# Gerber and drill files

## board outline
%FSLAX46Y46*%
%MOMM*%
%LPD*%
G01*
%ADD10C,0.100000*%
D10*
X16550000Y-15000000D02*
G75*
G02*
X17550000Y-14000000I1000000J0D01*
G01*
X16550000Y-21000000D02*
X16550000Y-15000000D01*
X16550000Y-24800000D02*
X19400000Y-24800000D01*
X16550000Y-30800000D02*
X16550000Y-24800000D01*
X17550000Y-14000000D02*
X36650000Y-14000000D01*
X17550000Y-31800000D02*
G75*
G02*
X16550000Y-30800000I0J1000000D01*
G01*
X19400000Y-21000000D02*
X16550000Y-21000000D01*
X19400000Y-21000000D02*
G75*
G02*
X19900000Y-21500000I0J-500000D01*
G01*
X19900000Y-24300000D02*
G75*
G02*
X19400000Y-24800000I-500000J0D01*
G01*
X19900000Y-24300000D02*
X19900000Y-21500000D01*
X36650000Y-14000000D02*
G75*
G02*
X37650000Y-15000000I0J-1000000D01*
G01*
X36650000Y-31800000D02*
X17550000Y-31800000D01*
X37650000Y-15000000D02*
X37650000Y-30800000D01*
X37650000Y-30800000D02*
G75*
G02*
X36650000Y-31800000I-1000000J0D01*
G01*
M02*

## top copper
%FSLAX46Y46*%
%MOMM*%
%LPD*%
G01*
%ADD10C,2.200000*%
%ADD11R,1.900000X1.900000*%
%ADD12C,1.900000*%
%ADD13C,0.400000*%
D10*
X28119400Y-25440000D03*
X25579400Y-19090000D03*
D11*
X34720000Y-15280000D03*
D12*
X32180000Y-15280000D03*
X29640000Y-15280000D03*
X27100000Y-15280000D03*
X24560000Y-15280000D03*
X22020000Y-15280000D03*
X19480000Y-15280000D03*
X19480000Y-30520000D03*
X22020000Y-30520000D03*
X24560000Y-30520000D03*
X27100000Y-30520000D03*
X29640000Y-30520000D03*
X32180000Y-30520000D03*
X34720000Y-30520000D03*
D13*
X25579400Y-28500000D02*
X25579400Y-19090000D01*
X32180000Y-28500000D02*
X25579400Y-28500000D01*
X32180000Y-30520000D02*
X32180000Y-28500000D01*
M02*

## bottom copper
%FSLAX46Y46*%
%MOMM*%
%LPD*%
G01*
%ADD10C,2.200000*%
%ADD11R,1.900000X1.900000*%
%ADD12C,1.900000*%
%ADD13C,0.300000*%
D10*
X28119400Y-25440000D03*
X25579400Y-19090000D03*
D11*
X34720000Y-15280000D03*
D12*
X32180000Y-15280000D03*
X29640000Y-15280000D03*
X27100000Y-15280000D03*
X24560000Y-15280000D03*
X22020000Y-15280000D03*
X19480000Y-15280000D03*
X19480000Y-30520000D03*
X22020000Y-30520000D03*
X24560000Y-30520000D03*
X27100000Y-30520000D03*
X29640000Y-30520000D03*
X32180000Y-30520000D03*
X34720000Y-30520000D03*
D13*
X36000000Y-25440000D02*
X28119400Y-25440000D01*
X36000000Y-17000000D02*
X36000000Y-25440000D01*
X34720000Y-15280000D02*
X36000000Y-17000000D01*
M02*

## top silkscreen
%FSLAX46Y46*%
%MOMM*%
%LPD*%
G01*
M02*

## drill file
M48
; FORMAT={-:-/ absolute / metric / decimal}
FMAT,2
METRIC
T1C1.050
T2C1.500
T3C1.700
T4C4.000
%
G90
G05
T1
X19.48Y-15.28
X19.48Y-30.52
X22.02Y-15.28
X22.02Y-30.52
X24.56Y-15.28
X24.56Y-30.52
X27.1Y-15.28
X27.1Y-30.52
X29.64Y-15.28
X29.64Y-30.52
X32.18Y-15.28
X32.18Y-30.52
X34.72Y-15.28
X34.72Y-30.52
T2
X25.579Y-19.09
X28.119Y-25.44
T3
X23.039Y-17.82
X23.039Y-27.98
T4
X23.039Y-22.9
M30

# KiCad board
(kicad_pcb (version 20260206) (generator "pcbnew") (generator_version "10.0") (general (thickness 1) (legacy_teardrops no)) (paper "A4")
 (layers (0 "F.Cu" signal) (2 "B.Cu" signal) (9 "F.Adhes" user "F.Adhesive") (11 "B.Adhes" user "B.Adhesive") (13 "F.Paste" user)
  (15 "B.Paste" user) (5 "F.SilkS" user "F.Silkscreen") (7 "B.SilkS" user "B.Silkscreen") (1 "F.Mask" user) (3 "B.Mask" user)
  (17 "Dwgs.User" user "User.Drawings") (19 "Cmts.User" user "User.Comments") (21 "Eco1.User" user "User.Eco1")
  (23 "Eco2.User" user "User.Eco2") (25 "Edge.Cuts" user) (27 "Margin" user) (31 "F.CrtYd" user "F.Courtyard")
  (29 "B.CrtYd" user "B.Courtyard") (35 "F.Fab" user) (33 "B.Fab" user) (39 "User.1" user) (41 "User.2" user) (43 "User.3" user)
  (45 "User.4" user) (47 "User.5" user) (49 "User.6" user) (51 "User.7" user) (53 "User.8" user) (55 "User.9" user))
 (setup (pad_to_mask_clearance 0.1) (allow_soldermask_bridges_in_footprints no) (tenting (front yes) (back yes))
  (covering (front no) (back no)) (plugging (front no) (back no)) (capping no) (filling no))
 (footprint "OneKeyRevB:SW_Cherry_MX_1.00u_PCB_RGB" (layer "F.Cu") (at 28.1194 25.44)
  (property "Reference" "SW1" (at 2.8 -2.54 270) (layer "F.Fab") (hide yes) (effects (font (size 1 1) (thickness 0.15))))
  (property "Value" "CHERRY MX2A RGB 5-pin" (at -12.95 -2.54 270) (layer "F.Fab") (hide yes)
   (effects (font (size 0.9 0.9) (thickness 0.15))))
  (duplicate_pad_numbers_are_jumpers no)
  (pad "" np_thru_hole circle (at -5.08 -7.62) (size 1.7 1.7) (drill 1.7) (layers "*.Cu" "*.Mask"))
  (pad "" np_thru_hole circle (at -5.08 -2.54) (size 4 4) (drill 4) (layers "*.Cu" "*.Mask"))
  (pad "" np_thru_hole circle (at -5.08 2.54) (size 1.7 1.7) (drill 1.7) (layers "*.Cu" "*.Mask"))
  (pad "1" thru_hole circle (at 0 0) (size 2.2 2.2) (drill 1.5) (layers "*.Cu" "*.Mask") (remove_unused_layers no) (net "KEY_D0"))
  (pad "2" thru_hole circle (at -2.54 -6.35) (size 2.2 2.2) (drill 1.5) (layers "*.Cu" "*.Mask") (remove_unused_layers no) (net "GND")))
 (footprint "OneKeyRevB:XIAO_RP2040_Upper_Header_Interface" (layer "F.Cu") (at 27.1 22.9)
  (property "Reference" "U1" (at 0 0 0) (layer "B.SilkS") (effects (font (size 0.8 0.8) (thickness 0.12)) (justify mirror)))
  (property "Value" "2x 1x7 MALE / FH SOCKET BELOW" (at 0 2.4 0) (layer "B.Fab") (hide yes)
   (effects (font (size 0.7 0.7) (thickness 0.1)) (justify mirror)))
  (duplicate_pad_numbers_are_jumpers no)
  (pad "1" thru_hole rect (at 7.62 -7.62) (size 1.9 1.9) (drill 1.05) (layers "*.Cu" "*.Mask") (remove_unused_layers no) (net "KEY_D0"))
  (pad "2" thru_hole circle (at 5.08 -7.62) (size 1.9 1.9) (drill 1.05) (layers "*.Cu" "*.Mask") (remove_unused_layers no))
  (pad "3" thru_hole circle (at 2.54 -7.62) (size 1.9 1.9) (drill 1.05) (layers "*.Cu" "*.Mask") (remove_unused_layers no))
  (pad "4" thru_hole circle (at 0 -7.62) (size 1.9 1.9) (drill 1.05) (layers "*.Cu" "*.Mask") (remove_unused_layers no))
  (pad "5" thru_hole circle (at -2.54 -7.62) (size 1.9 1.9) (drill 1.05) (layers "*.Cu" "*.Mask") (remove_unused_layers no))
  (pad "6" thru_hole circle (at -5.08 -7.62) (size 1.9 1.9) (drill 1.05) (layers "*.Cu" "*.Mask") (remove_unused_layers no))
  (pad "7" thru_hole circle (at -7.62 -7.62) (size 1.9 1.9) (drill 1.05) (layers "*.Cu" "*.Mask") (remove_unused_layers no))
  (pad "8" thru_hole circle (at -7.62 7.62) (size 1.9 1.9) (drill 1.05) (layers "*.Cu" "*.Mask") (remove_unused_layers no))
  (pad "9" thru_hole circle (at -5.08 7.62) (size 1.9 1.9) (drill 1.05) (layers "*.Cu" "*.Mask") (remove_unused_layers no))
  (pad "10" thru_hole circle (at -2.54 7.62) (size 1.9 1.9) (drill 1.05) (layers "*.Cu" "*.Mask") (remove_unused_layers no))
  (pad "11" thru_hole circle (at 0 7.62) (size 1.9 1.9) (drill 1.05) (layers "*.Cu" "*.Mask") (remove_unused_layers no))
  (pad "12" thru_hole circle (at 2.54 7.62) (size 1.9 1.9) (drill 1.05) (layers "*.Cu" "*.Mask") (remove_unused_layers no))
  (pad "13" thru_hole circle (at 5.08 7.62) (size 1.9 1.9) (drill 1.05) (layers "*.Cu" "*.Mask") (remove_unused_layers no) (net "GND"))
  (pad "14" thru_hole circle (at 7.62 7.62) (size 1.9 1.9) (drill 1.05) (layers "*.Cu" "*.Mask") (remove_unused_layers no)))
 (gr_arc (start 16.55 15) (mid 16.842893 14.292893) (end 17.55 14) (stroke (width 0.1) (type solid)) (layer "Edge.Cuts"))
 (gr_line (start 16.55 21) (end 16.55 15) (stroke (width 0.1) (type solid)) (layer "Edge.Cuts"))
 (gr_line (start 16.55 24.8) (end 19.4 24.8) (stroke (width 0.1) (type solid)) (layer "Edge.Cuts"))
 (gr_line (start 16.55 30.8) (end 16.55 24.8) (stroke (width 0.1) (type solid)) (layer "Edge.Cuts"))
 (gr_line (start 17.55 14) (end 36.65 14) (stroke (width 0.1) (type solid)) (layer "Edge.Cuts"))
 (gr_arc (start 17.55 31.8) (mid 16.842893 31.507107) (end 16.55 30.8) (stroke (width 0.1) (type solid)) (layer "Edge.Cuts"))
 (gr_line (start 19.4 21) (end 16.55 21) (stroke (width 0.1) (type solid)) (layer "Edge.Cuts"))
 (gr_arc (start 19.4 21) (mid 19.753553 21.146447) (end 19.9 21.5) (stroke (width 0.1) (type solid)) (layer "Edge.Cuts"))
 (gr_arc (start 19.9 24.3) (mid 19.753553 24.653553) (end 19.4 24.8) (stroke (width 0.1) (type solid)) (layer "Edge.Cuts"))
 (gr_line (start 19.9 24.3) (end 19.9 21.5) (stroke (width 0.1) (type solid)) (layer "Edge.Cuts"))
 (gr_arc (start 36.65 14) (mid 37.357107 14.292893) (end 37.65 15) (stroke (width 0.1) (type solid)) (layer "Edge.Cuts"))
 (gr_line (start 36.65 31.8) (end 17.55 31.8) (stroke (width 0.1) (type solid)) (layer "Edge.Cuts"))
 (gr_line (start 37.65 15) (end 37.65 30.8) (stroke (width 0.1) (type solid)) (layer "Edge.Cuts"))
 (gr_arc (start 37.65 30.8) (mid 37.357107 31.507107) (end 36.65 31.8) (stroke (width 0.1) (type solid)) (layer "Edge.Cuts"))
 (segment (start 36 25.44) (end 28.1194 25.44) (width 0.3) (layer "B.Cu") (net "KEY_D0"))
 (segment (start 36 17) (end 36 25.44) (width 0.3) (layer "B.Cu") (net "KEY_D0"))
 (segment (start 34.72 15.28) (end 36 17) (width 0.3) (layer "B.Cu") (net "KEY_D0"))
 (segment (start 25.5794 28.5) (end 25.5794 19.09) (width 0.4) (layer "F.Cu") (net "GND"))
 (segment (start 32.18 28.5) (end 25.5794 28.5) (width 0.4) (layer "F.Cu") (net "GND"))
 (segment (start 32.18 30.52) (end 32.18 28.5) (width 0.4) (layer "F.Cu") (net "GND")))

